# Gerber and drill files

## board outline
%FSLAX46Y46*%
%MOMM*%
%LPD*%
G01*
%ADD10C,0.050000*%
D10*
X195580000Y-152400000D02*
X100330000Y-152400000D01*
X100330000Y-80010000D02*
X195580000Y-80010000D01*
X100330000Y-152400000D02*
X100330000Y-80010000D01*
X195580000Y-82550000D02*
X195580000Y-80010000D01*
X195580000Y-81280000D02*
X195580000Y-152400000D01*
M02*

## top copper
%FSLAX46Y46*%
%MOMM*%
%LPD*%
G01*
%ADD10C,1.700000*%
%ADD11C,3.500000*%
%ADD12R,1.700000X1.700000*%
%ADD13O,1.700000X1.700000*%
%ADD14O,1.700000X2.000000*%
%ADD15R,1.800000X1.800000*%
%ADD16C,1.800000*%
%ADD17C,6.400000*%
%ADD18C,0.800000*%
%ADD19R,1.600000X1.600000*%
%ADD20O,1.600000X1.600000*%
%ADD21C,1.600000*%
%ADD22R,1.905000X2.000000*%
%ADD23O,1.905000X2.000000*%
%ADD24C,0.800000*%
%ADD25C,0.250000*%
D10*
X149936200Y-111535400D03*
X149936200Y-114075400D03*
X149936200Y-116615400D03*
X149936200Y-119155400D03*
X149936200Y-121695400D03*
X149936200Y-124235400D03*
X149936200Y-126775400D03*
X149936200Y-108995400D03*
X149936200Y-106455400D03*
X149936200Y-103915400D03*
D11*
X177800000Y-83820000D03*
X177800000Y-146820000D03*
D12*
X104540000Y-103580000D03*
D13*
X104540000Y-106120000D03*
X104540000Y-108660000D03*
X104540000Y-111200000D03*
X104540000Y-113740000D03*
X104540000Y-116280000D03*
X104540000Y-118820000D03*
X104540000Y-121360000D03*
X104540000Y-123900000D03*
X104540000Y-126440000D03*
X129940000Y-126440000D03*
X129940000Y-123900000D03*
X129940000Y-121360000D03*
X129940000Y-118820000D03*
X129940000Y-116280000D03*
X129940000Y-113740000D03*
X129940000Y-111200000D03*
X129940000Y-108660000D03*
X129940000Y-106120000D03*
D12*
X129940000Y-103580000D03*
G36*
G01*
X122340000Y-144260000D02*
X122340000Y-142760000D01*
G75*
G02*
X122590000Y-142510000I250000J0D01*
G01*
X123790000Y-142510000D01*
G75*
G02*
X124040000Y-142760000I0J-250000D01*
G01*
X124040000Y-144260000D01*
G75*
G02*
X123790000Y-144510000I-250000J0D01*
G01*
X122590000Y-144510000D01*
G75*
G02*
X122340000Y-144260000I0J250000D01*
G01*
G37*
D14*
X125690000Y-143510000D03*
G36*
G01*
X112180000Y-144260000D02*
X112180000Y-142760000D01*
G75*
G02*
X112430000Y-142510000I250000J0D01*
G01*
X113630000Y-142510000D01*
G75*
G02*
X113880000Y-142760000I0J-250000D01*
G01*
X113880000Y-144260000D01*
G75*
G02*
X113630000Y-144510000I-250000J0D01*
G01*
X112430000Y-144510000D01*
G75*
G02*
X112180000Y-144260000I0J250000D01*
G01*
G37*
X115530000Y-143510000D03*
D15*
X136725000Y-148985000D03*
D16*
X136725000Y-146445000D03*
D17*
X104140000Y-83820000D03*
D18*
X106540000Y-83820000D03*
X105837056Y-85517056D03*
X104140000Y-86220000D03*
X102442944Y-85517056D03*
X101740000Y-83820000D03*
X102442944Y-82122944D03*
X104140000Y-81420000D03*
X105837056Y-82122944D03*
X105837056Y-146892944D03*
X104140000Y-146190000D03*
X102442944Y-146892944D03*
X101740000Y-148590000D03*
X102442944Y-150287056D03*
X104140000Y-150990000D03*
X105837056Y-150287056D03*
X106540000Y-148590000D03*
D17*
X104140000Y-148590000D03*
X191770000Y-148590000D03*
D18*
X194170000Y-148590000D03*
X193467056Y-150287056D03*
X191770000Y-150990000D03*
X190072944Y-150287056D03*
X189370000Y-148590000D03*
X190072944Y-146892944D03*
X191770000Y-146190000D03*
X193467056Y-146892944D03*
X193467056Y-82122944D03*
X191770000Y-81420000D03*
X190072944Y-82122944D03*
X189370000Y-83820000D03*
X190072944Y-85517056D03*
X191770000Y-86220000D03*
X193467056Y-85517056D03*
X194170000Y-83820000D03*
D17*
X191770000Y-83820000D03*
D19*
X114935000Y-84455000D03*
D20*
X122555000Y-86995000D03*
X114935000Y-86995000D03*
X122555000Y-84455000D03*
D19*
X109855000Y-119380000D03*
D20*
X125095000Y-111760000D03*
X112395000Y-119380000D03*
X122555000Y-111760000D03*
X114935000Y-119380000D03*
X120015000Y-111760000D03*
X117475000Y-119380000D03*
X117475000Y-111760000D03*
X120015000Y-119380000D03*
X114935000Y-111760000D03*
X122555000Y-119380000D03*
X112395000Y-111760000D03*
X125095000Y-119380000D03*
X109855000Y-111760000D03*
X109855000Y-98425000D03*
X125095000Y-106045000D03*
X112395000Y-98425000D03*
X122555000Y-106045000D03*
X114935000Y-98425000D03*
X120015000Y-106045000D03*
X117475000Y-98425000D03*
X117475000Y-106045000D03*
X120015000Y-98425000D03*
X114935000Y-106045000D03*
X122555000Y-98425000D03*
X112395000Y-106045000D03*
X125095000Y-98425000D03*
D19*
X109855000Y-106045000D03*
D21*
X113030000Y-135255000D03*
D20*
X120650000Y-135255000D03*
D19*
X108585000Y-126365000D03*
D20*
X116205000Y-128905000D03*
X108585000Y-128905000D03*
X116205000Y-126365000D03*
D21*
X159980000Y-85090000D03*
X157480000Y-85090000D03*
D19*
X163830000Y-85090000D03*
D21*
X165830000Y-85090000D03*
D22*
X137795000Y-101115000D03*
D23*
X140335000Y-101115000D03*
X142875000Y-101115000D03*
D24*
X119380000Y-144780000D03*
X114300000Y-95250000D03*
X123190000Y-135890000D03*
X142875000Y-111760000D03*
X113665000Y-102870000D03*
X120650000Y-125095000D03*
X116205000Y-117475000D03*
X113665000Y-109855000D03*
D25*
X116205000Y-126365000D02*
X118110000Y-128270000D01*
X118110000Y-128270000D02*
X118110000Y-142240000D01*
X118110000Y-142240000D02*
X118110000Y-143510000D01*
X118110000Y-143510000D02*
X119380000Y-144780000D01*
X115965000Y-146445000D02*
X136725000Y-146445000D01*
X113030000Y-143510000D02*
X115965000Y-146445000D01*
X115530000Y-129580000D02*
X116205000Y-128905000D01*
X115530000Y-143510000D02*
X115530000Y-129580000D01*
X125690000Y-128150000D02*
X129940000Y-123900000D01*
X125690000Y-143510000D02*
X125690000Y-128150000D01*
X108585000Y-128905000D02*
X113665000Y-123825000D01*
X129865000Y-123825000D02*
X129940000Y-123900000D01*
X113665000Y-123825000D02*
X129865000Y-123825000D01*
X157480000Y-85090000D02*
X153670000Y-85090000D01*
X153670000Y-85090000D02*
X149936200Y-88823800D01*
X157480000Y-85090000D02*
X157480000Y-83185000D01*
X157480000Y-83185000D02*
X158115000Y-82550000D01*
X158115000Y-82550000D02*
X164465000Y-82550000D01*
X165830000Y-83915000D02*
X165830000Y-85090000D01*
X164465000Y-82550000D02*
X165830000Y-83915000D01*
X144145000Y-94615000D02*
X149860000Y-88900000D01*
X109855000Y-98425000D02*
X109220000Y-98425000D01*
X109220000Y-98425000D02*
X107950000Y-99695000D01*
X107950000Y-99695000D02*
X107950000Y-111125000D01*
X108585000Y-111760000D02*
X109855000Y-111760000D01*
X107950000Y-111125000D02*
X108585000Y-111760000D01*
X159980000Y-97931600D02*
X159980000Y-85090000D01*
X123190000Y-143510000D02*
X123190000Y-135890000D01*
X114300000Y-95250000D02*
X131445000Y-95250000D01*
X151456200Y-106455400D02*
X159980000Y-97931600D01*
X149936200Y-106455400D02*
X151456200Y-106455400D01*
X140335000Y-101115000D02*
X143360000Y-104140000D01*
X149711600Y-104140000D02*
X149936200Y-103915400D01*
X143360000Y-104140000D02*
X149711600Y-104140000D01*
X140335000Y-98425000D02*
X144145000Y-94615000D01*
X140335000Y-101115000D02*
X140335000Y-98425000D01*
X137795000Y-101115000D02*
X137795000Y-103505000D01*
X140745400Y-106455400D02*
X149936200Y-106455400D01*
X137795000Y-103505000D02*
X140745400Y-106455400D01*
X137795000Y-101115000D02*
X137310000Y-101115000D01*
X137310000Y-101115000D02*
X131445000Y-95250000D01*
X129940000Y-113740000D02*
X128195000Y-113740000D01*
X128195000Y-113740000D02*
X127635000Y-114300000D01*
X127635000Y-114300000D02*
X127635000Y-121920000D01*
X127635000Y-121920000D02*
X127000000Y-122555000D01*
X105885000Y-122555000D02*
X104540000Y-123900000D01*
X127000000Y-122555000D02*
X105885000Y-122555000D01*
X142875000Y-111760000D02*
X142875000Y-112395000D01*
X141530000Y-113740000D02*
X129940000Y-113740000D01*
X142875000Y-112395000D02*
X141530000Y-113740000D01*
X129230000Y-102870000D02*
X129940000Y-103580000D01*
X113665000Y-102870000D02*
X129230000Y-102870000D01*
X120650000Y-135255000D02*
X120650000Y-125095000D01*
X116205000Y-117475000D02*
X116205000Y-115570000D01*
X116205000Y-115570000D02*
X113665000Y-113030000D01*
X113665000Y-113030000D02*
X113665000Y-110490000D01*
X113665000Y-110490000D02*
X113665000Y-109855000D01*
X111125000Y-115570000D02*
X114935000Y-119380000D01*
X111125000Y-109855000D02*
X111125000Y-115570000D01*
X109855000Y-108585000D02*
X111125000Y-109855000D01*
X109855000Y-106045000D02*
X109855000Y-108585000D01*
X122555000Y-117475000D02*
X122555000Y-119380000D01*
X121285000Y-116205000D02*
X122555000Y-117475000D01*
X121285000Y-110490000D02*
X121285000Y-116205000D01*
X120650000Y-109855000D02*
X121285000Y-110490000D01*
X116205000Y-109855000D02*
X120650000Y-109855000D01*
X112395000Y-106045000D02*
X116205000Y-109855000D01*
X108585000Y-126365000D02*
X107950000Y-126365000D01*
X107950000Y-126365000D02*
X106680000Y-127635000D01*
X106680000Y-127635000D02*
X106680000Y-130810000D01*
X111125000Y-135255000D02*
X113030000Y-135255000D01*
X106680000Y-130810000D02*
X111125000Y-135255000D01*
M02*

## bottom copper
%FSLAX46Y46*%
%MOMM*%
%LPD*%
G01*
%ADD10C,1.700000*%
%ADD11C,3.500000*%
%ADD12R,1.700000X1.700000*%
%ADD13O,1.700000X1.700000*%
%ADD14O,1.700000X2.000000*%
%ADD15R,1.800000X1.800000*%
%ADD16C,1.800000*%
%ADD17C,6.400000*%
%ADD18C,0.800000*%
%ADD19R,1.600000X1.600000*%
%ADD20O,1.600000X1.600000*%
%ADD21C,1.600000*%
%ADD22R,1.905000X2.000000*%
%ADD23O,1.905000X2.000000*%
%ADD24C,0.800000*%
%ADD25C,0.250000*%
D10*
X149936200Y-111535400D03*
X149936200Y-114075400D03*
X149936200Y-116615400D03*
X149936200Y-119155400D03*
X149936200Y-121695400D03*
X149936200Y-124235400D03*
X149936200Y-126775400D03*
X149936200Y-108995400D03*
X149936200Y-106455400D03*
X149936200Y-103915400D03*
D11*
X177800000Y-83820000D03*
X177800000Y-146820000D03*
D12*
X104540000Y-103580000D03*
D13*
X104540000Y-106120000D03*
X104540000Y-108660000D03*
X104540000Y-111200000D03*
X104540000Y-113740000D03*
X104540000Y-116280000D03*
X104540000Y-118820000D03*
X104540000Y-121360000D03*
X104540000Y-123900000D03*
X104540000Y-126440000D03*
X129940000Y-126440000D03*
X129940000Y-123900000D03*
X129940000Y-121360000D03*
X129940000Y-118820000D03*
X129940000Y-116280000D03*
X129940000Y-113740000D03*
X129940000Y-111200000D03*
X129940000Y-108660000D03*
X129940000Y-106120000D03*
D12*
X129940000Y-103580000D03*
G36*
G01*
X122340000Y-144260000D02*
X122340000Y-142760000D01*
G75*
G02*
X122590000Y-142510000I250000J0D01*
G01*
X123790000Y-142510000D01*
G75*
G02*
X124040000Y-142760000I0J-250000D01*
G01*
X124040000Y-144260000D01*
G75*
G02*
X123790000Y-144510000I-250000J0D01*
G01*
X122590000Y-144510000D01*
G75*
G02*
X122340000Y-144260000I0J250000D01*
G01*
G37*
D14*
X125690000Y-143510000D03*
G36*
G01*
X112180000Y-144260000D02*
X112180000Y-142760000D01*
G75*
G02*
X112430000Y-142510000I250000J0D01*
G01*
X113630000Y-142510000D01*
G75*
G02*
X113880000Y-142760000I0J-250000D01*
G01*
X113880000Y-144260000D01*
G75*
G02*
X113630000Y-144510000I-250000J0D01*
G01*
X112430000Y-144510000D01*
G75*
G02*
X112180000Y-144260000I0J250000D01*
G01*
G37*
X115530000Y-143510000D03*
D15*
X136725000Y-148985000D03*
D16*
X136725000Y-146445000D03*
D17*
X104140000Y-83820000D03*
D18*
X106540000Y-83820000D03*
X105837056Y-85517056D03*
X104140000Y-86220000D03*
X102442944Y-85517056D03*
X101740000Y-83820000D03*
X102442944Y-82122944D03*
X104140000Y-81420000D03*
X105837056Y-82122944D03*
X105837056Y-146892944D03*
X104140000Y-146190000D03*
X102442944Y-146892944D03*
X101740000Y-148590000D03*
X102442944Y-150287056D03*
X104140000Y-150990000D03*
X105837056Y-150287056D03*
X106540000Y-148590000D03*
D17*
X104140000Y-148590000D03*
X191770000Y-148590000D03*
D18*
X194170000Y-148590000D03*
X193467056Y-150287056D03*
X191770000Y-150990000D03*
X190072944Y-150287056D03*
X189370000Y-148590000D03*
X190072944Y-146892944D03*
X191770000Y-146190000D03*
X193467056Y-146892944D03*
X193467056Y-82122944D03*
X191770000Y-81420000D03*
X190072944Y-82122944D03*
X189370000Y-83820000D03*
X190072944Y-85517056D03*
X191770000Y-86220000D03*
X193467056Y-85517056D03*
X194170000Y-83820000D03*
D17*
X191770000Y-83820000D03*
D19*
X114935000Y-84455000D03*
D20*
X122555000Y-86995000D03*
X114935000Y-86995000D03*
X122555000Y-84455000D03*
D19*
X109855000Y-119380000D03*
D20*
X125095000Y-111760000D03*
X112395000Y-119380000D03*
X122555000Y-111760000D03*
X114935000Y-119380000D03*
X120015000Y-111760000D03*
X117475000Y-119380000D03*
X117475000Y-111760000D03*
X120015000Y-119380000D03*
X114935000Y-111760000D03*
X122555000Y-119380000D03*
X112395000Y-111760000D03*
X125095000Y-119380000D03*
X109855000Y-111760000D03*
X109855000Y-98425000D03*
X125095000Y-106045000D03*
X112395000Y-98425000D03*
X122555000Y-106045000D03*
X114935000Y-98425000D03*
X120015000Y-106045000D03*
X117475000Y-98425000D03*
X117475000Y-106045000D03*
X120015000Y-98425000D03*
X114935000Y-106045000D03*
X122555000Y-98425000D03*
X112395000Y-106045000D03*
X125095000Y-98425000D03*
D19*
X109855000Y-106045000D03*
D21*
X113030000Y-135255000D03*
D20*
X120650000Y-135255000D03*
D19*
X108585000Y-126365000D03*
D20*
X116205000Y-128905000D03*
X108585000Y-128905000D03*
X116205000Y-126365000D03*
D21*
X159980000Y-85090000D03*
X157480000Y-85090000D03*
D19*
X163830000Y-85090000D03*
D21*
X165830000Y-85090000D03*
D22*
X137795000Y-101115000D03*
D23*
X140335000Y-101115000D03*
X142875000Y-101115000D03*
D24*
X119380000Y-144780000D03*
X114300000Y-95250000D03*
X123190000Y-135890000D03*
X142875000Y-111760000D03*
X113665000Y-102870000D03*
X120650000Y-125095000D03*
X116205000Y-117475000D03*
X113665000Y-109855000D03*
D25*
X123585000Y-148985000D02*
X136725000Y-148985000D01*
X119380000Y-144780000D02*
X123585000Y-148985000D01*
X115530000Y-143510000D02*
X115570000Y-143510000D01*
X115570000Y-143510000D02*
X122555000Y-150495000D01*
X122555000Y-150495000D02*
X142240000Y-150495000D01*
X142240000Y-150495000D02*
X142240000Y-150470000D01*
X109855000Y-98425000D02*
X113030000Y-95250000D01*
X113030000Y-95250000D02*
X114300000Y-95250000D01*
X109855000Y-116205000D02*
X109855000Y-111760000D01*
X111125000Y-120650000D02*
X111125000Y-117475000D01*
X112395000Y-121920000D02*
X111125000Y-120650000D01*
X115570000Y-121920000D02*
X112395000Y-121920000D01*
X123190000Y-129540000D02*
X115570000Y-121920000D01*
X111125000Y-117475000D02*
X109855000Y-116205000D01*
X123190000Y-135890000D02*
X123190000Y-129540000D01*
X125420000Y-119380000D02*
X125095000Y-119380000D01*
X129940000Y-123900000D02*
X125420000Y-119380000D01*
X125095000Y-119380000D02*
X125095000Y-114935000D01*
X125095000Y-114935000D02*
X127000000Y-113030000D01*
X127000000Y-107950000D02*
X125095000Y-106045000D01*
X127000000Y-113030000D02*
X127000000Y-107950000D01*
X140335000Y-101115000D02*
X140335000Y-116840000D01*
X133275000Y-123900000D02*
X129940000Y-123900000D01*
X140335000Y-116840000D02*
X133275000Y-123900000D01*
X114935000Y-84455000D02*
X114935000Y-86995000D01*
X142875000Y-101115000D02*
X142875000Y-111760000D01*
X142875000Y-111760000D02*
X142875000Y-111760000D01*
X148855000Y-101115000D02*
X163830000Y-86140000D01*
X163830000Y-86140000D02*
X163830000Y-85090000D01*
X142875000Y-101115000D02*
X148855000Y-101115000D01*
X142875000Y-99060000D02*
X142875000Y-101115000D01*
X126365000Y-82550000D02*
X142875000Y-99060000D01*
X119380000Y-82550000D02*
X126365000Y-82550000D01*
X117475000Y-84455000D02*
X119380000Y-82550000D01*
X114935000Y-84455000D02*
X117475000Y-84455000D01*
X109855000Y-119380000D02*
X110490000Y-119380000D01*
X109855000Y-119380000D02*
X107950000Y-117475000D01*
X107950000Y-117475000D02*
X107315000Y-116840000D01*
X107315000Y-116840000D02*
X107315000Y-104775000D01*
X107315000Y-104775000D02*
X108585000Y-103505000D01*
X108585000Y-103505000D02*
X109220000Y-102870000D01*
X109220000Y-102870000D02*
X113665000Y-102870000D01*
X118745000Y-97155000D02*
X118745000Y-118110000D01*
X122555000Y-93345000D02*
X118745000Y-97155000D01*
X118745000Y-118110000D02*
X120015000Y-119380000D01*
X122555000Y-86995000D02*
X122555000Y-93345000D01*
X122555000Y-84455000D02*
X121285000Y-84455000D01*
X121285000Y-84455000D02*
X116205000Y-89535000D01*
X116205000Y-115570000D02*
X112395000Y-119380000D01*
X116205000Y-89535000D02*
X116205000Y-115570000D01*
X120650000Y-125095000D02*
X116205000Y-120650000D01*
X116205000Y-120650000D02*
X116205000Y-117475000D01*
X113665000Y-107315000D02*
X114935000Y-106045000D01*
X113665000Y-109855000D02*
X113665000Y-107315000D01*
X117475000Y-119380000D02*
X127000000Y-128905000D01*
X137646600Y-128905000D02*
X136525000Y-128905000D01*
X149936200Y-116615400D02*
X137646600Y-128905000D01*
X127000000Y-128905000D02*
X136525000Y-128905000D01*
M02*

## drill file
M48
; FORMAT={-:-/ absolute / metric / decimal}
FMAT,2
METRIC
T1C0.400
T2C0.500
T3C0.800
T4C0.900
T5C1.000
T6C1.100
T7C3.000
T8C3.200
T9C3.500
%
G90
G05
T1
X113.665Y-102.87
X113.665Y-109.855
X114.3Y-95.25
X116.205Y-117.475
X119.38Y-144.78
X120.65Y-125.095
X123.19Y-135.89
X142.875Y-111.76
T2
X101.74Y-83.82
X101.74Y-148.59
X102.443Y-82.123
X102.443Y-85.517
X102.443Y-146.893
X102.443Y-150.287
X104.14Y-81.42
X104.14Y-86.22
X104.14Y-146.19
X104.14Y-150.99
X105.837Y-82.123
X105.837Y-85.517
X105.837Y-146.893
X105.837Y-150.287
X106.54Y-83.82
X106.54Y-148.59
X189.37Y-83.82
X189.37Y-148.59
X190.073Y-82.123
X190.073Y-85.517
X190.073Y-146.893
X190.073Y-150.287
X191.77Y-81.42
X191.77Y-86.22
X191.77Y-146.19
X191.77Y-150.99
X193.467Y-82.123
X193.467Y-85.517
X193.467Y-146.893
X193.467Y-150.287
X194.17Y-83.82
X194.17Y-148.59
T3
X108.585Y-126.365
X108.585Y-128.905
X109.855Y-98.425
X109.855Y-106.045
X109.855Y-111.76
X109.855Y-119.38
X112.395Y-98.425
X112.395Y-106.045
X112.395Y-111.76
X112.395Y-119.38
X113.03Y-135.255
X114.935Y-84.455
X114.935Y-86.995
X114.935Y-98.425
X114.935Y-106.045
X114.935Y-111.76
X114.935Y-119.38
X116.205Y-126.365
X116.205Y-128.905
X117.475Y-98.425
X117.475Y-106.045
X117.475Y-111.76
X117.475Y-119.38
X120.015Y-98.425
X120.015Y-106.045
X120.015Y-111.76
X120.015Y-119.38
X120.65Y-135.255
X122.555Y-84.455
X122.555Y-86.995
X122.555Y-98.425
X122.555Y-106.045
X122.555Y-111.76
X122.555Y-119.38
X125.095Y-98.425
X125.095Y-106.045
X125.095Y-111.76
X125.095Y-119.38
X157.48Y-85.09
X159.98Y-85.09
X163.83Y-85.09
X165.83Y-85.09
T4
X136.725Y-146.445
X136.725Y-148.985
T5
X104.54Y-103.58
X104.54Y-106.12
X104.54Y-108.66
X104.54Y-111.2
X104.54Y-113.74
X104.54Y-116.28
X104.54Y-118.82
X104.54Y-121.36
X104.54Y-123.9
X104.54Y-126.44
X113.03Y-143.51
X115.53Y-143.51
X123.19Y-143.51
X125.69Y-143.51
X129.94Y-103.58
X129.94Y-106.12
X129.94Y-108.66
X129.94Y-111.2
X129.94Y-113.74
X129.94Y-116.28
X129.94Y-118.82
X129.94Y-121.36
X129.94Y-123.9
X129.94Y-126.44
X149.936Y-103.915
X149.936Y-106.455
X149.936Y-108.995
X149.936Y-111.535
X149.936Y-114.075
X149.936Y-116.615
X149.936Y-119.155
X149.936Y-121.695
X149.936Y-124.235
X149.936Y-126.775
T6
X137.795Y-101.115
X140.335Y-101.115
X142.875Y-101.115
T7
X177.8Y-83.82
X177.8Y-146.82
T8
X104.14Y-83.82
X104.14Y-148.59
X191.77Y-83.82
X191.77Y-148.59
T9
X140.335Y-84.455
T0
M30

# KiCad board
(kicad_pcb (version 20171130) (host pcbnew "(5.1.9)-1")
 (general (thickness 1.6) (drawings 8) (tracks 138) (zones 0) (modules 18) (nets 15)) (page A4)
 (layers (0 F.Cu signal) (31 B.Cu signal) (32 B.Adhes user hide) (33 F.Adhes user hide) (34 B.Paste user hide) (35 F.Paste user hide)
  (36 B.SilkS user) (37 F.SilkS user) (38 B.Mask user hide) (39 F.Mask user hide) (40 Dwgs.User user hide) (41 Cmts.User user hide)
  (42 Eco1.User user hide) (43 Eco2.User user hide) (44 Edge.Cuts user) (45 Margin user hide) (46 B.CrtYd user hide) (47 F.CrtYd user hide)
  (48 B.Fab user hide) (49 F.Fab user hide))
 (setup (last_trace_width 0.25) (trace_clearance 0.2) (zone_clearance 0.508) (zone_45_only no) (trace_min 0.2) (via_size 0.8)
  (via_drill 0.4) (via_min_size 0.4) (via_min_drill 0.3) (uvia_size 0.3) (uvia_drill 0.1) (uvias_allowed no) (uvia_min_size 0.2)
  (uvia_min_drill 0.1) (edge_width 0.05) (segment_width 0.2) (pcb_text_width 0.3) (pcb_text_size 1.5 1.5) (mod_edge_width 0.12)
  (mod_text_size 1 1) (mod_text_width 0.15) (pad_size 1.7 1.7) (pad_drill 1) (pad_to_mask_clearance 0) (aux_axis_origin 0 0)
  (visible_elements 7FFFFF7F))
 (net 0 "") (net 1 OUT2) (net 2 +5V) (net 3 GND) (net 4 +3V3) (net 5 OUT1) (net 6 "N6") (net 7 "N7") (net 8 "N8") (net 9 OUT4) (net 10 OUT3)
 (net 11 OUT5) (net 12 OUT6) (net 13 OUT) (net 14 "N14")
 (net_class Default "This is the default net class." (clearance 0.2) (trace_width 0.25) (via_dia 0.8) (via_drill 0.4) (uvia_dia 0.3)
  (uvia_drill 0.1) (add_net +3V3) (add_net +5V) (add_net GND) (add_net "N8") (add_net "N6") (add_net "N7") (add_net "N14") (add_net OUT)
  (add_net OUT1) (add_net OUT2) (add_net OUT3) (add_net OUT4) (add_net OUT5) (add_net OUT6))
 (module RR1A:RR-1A (layer F.Cu) (at 177.8 115.32 270)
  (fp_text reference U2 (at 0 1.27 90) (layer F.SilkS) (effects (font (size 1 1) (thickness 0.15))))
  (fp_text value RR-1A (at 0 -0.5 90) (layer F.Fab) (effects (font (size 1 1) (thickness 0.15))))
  (pad 4 thru_hole circle (at -3.7846 27.8638 270) (size 1.7 1.7) (drill 1) (layers *.Cu *.Mask))
  (pad 5 thru_hole circle (at -1.2446 27.8638 270) (size 1.7 1.7) (drill 1) (layers *.Cu *.Mask))
  (pad 6 thru_hole circle (at 1.2954 27.8638 270) (size 1.7 1.7) (drill 1) (layers *.Cu *.Mask) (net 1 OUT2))
  (pad 7 thru_hole circle (at 3.8354 27.8638 270) (size 1.7 1.7) (drill 1) (layers *.Cu *.Mask))
  (pad 8 thru_hole circle (at 6.3754 27.8638 270) (size 1.7 1.7) (drill 1) (layers *.Cu *.Mask))
  (pad 9 thru_hole circle (at 8.9154 27.8638 270) (size 1.7 1.7) (drill 1) (layers *.Cu *.Mask))
  (pad 10 thru_hole circle (at 11.4554 27.8638 270) (size 1.7 1.7) (drill 1) (layers *.Cu *.Mask))
  (pad 3 thru_hole circle (at -6.3246 27.8638 270) (size 1.7 1.7) (drill 1) (layers *.Cu *.Mask))
  (pad 2 thru_hole circle (at -8.8646 27.8638 270) (size 1.7 1.7) (drill 1) (layers *.Cu *.Mask) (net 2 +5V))
  (pad 1 thru_hole circle (at -11.4046 27.8638 270) (size 1.7 1.7) (drill 1) (layers *.Cu *.Mask) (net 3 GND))
  (pad 11 thru_hole circle (at -31.5 0 270) (size 3.5 3.5) (drill 3) (layers *.Cu *.Mask))
  (pad 12 thru_hole circle (at 31.5 0 270) (size 3.5 3.5) (drill 3) (layers *.Cu *.Mask)))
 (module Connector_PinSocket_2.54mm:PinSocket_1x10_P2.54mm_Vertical (layer F.Cu) (at 104.54 103.58)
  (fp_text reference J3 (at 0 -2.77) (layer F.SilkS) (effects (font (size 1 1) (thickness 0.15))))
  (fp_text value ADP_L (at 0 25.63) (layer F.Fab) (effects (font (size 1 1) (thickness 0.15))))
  (pad 1 thru_hole rect (at 0 0) (size 1.7 1.7) (drill 1) (layers *.Cu *.Mask))
  (pad 2 thru_hole oval (at 0 2.54) (size 1.7 1.7) (drill 1) (layers *.Cu *.Mask))
  (pad 3 thru_hole oval (at 0 5.08) (size 1.7 1.7) (drill 1) (layers *.Cu *.Mask))
  (pad 4 thru_hole oval (at 0 7.62) (size 1.7 1.7) (drill 1) (layers *.Cu *.Mask))
  (pad 5 thru_hole oval (at 0 10.16) (size 1.7 1.7) (drill 1) (layers *.Cu *.Mask))
  (pad 6 thru_hole oval (at 0 12.7) (size 1.7 1.7) (drill 1) (layers *.Cu *.Mask))
  (pad 7 thru_hole oval (at 0 15.24) (size 1.7 1.7) (drill 1) (layers *.Cu *.Mask))
  (pad 8 thru_hole oval (at 0 17.78) (size 1.7 1.7) (drill 1) (layers *.Cu *.Mask))
  (pad 9 thru_hole oval (at 0 20.32) (size 1.7 1.7) (drill 1) (layers *.Cu *.Mask) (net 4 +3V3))
  (pad 10 thru_hole oval (at 0 22.86) (size 1.7 1.7) (drill 1) (layers *.Cu *.Mask)))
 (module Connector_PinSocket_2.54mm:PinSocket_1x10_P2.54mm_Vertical (layer F.Cu) (at 129.94 103.58)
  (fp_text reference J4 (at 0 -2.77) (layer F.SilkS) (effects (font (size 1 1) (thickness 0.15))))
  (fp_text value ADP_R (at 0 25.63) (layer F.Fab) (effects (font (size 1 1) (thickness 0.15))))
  (pad 10 thru_hole oval (at 0 22.86) (size 1.7 1.7) (drill 1) (layers *.Cu *.Mask))
  (pad 9 thru_hole oval (at 0 20.32) (size 1.7 1.7) (drill 1) (layers *.Cu *.Mask) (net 3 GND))
  (pad 8 thru_hole oval (at 0 17.78) (size 1.7 1.7) (drill 1) (layers *.Cu *.Mask))
  (pad 7 thru_hole oval (at 0 15.24) (size 1.7 1.7) (drill 1) (layers *.Cu *.Mask))
  (pad 6 thru_hole oval (at 0 12.7) (size 1.7 1.7) (drill 1) (layers *.Cu *.Mask))
  (pad 5 thru_hole oval (at 0 10.16) (size 1.7 1.7) (drill 1) (layers *.Cu *.Mask) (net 4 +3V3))
  (pad 4 thru_hole oval (at 0 7.62) (size 1.7 1.7) (drill 1) (layers *.Cu *.Mask))
  (pad 3 thru_hole oval (at 0 5.08) (size 1.7 1.7) (drill 1) (layers *.Cu *.Mask))
  (pad 2 thru_hole oval (at 0 2.54) (size 1.7 1.7) (drill 1) (layers *.Cu *.Mask))
  (pad 1 thru_hole rect (at 0 0) (size 1.7 1.7) (drill 1) (layers *.Cu *.Mask) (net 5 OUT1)))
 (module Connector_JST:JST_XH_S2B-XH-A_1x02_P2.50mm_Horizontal (layer F.Cu) (at 123.19 143.51)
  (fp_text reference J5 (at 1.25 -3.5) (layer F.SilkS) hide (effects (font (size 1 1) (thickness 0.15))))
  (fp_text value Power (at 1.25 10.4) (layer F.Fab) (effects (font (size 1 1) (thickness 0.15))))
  (pad 1 thru_hole roundrect (at 0 0) (size 1.7 2) (drill 1) (layers *.Cu *.Mask) (roundrect_rratio 0.1470588235294118) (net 2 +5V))
  (pad 2 thru_hole oval (at 2.5 0) (size 1.7 2) (drill 1) (layers *.Cu *.Mask) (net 3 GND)))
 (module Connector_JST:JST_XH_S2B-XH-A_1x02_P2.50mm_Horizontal (layer F.Cu) (at 113.03 143.51)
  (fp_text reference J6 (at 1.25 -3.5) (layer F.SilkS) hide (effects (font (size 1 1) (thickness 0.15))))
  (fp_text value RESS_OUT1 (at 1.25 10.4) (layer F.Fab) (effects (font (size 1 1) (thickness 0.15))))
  (pad 1 thru_hole roundrect (at 0 0) (size 1.7 2) (drill 1) (layers *.Cu *.Mask) (roundrect_rratio 0.1470588235294118) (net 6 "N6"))
  (pad 2 thru_hole oval (at 2.5 0) (size 1.7 2) (drill 1) (layers *.Cu *.Mask) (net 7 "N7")))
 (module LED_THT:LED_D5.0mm (layer F.Cu) (at 136.725 148.985 90)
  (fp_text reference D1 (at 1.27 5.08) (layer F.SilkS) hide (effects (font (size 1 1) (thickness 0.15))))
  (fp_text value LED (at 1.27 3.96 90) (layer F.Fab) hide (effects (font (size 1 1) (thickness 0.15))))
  (pad 1 thru_hole rect (at 0 0 90) (size 1.8 1.8) (drill 0.9) (layers *.Cu *.Mask) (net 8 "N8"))
  (pad 2 thru_hole circle (at 2.54 0 90) (size 1.8 1.8) (drill 0.9) (layers *.Cu *.Mask) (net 6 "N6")))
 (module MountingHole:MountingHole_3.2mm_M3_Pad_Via (layer F.Cu) (at 104.14 83.82)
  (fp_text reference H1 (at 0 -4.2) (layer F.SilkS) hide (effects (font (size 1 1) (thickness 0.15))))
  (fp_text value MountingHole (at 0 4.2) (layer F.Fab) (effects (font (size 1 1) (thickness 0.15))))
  (pad 1 thru_hole circle (at 0 0) (size 6.4 6.4) (drill 3.2) (layers *.Cu *.Mask))
  (pad 1 thru_hole circle (at 2.4 0) (size 0.8 0.8) (drill 0.5) (layers *.Cu *.Mask))
  (pad 1 thru_hole circle (at 1.697056 1.697056) (size 0.8 0.8) (drill 0.5) (layers *.Cu *.Mask))
  (pad 1 thru_hole circle (at 0 2.4) (size 0.8 0.8) (drill 0.5) (layers *.Cu *.Mask))
  (pad 1 thru_hole circle (at -1.697056 1.697056) (size 0.8 0.8) (drill 0.5) (layers *.Cu *.Mask))
  (pad 1 thru_hole circle (at -2.4 0) (size 0.8 0.8) (drill 0.5) (layers *.Cu *.Mask))
  (pad 1 thru_hole circle (at -1.697056 -1.697056) (size 0.8 0.8) (drill 0.5) (layers *.Cu *.Mask))
  (pad 1 thru_hole circle (at 0 -2.4) (size 0.8 0.8) (drill 0.5) (layers *.Cu *.Mask))
  (pad 1 thru_hole circle (at 1.697056 -1.697056) (size 0.8 0.8) (drill 0.5) (layers *.Cu *.Mask)))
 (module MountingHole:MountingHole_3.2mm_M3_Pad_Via (layer F.Cu) (at 104.14 148.59)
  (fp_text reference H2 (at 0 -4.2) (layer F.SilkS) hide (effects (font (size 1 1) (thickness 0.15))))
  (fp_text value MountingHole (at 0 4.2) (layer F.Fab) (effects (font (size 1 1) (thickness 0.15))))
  (pad 1 thru_hole circle (at 1.697056 -1.697056) (size 0.8 0.8) (drill 0.5) (layers *.Cu *.Mask))
  (pad 1 thru_hole circle (at 0 -2.4) (size 0.8 0.8) (drill 0.5) (layers *.Cu *.Mask))
  (pad 1 thru_hole circle (at -1.697056 -1.697056) (size 0.8 0.8) (drill 0.5) (layers *.Cu *.Mask))
  (pad 1 thru_hole circle (at -2.4 0) (size 0.8 0.8) (drill 0.5) (layers *.Cu *.Mask))
  (pad 1 thru_hole circle (at -1.697056 1.697056) (size 0.8 0.8) (drill 0.5) (layers *.Cu *.Mask))
  (pad 1 thru_hole circle (at 0 2.4) (size 0.8 0.8) (drill 0.5) (layers *.Cu *.Mask))
  (pad 1 thru_hole circle (at 1.697056 1.697056) (size 0.8 0.8) (drill 0.5) (layers *.Cu *.Mask))
  (pad 1 thru_hole circle (at 2.4 0) (size 0.8 0.8) (drill 0.5) (layers *.Cu *.Mask))
  (pad 1 thru_hole circle (at 0 0) (size 6.4 6.4) (drill 3.2) (layers *.Cu *.Mask)))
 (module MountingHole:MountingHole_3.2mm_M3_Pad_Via (layer F.Cu) (at 191.77 148.59)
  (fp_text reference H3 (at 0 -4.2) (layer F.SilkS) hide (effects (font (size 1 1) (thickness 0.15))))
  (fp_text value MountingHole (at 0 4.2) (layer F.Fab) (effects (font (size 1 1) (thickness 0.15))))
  (pad 1 thru_hole circle (at 0 0) (size 6.4 6.4) (drill 3.2) (layers *.Cu *.Mask))
  (pad 1 thru_hole circle (at 2.4 0) (size 0.8 0.8) (drill 0.5) (layers *.Cu *.Mask))
  (pad 1 thru_hole circle (at 1.697056 1.697056) (size 0.8 0.8) (drill 0.5) (layers *.Cu *.Mask))
  (pad 1 thru_hole circle (at 0 2.4) (size 0.8 0.8) (drill 0.5) (layers *.Cu *.Mask))
  (pad 1 thru_hole circle (at -1.697056 1.697056) (size 0.8 0.8) (drill 0.5) (layers *.Cu *.Mask))
  (pad 1 thru_hole circle (at -2.4 0) (size 0.8 0.8) (drill 0.5) (layers *.Cu *.Mask))
  (pad 1 thru_hole circle (at -1.697056 -1.697056) (size 0.8 0.8) (drill 0.5) (layers *.Cu *.Mask))
  (pad 1 thru_hole circle (at 0 -2.4) (size 0.8 0.8) (drill 0.5) (layers *.Cu *.Mask))
  (pad 1 thru_hole circle (at 1.697056 -1.697056) (size 0.8 0.8) (drill 0.5) (layers *.Cu *.Mask)))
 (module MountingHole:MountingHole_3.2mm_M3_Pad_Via (layer F.Cu) (at 191.77 83.82)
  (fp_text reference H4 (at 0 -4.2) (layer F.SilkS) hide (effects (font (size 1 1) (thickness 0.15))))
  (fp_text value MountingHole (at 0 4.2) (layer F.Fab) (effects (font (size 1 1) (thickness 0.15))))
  (pad 1 thru_hole circle (at 1.697056 -1.697056) (size 0.8 0.8) (drill 0.5) (layers *.Cu *.Mask))
  (pad 1 thru_hole circle (at 0 -2.4) (size 0.8 0.8) (drill 0.5) (layers *.Cu *.Mask))
  (pad 1 thru_hole circle (at -1.697056 -1.697056) (size 0.8 0.8) (drill 0.5) (layers *.Cu *.Mask))
  (pad 1 thru_hole circle (at -2.4 0) (size 0.8 0.8) (drill 0.5) (layers *.Cu *.Mask))
  (pad 1 thru_hole circle (at -1.697056 1.697056) (size 0.8 0.8) (drill 0.5) (layers *.Cu *.Mask))
  (pad 1 thru_hole circle (at 0 2.4) (size 0.8 0.8) (drill 0.5) (layers *.Cu *.Mask))
  (pad 1 thru_hole circle (at 1.697056 1.697056) (size 0.8 0.8) (drill 0.5) (layers *.Cu *.Mask))
  (pad 1 thru_hole circle (at 2.4 0) (size 0.8 0.8) (drill 0.5) (layers *.Cu *.Mask))
  (pad 1 thru_hole circle (at 0 0) (size 6.4 6.4) (drill 3.2) (layers *.Cu *.Mask)))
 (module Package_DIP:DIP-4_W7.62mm (layer F.Cu) (at 114.935 84.455)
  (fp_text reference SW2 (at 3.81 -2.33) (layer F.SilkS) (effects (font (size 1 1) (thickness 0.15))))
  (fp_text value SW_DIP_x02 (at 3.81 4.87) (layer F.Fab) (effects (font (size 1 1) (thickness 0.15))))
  (pad 1 thru_hole rect (at 0 0) (size 1.6 1.6) (drill 0.8) (layers *.Cu *.Mask) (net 4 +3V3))
  (pad 3 thru_hole oval (at 7.62 2.54) (size 1.6 1.6) (drill 0.8) (layers *.Cu *.Mask) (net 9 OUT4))
  (pad 2 thru_hole oval (at 0 2.54) (size 1.6 1.6) (drill 0.8) (layers *.Cu *.Mask) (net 4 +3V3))
  (pad 4 thru_hole oval (at 7.62 0) (size 1.6 1.6) (drill 0.8) (layers *.Cu *.Mask) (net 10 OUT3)))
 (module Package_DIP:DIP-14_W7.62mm (layer F.Cu) (at 109.855 119.38 90)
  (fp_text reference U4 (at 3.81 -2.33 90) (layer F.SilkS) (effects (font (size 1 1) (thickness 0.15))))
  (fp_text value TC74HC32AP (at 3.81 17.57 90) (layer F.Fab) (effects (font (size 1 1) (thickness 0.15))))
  (pad 1 thru_hole rect (at 0 0 90) (size 1.6 1.6) (drill 0.8) (layers *.Cu *.Mask) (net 5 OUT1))
  (pad 8 thru_hole oval (at 7.62 15.24 90) (size 1.6 1.6) (drill 0.8) (layers *.Cu *.Mask))
  (pad 2 thru_hole oval (at 0 2.54 90) (size 1.6 1.6) (drill 0.8) (layers *.Cu *.Mask) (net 10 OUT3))
  (pad 9 thru_hole oval (at 7.62 12.7 90) (size 1.6 1.6) (drill 0.8) (layers *.Cu *.Mask))
  (pad 3 thru_hole oval (at 0 5.08 90) (size 1.6 1.6) (drill 0.8) (layers *.Cu *.Mask) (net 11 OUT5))
  (pad 10 thru_hole oval (at 7.62 10.16 90) (size 1.6 1.6) (drill 0.8) (layers *.Cu *.Mask))
  (pad 4 thru_hole oval (at 0 7.62 90) (size 1.6 1.6) (drill 0.8) (layers *.Cu *.Mask) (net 1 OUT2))
  (pad 11 thru_hole oval (at 7.62 7.62 90) (size 1.6 1.6) (drill 0.8) (layers *.Cu *.Mask))
  (pad 5 thru_hole oval (at 0 10.16 90) (size 1.6 1.6) (drill 0.8) (layers *.Cu *.Mask) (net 9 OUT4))
  (pad 12 thru_hole oval (at 7.62 5.08 90) (size 1.6 1.6) (drill 0.8) (layers *.Cu *.Mask))
  (pad 6 thru_hole oval (at 0 12.7 90) (size 1.6 1.6) (drill 0.8) (layers *.Cu *.Mask) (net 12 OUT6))
  (pad 13 thru_hole oval (at 7.62 2.54 90) (size 1.6 1.6) (drill 0.8) (layers *.Cu *.Mask))
  (pad 7 thru_hole oval (at 0 15.24 90) (size 1.6 1.6) (drill 0.8) (layers *.Cu *.Mask) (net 3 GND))
  (pad 14 thru_hole oval (at 7.62 0 90) (size 1.6 1.6) (drill 0.8) (layers *.Cu *.Mask) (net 2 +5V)))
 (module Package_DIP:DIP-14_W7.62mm (layer F.Cu) (at 109.855 106.045 90)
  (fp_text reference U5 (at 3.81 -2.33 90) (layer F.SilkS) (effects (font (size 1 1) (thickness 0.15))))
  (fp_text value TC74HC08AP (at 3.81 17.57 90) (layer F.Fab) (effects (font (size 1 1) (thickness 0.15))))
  (pad 14 thru_hole oval (at 7.62 0 90) (size 1.6 1.6) (drill 0.8) (layers *.Cu *.Mask) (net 2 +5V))
  (pad 7 thru_hole oval (at 0 15.24 90) (size 1.6 1.6) (drill 0.8) (layers *.Cu *.Mask) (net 3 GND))
  (pad 13 thru_hole oval (at 7.62 2.54 90) (size 1.6 1.6) (drill 0.8) (layers *.Cu *.Mask))
  (pad 6 thru_hole oval (at 0 12.7 90) (size 1.6 1.6) (drill 0.8) (layers *.Cu *.Mask))
  (pad 12 thru_hole oval (at 7.62 5.08 90) (size 1.6 1.6) (drill 0.8) (layers *.Cu *.Mask))
  (pad 5 thru_hole oval (at 0 10.16 90) (size 1.6 1.6) (drill 0.8) (layers *.Cu *.Mask))
  (pad 11 thru_hole oval (at 7.62 7.62 90) (size 1.6 1.6) (drill 0.8) (layers *.Cu *.Mask))
  (pad 4 thru_hole oval (at 0 7.62 90) (size 1.6 1.6) (drill 0.8) (layers *.Cu *.Mask))
  (pad 10 thru_hole oval (at 7.62 10.16 90) (size 1.6 1.6) (drill 0.8) (layers *.Cu *.Mask))
  (pad 3 thru_hole oval (at 0 5.08 90) (size 1.6 1.6) (drill 0.8) (layers *.Cu *.Mask) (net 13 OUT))
  (pad 9 thru_hole oval (at 7.62 12.7 90) (size 1.6 1.6) (drill 0.8) (layers *.Cu *.Mask))
  (pad 2 thru_hole oval (at 0 2.54 90) (size 1.6 1.6) (drill 0.8) (layers *.Cu *.Mask) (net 12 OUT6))
  (pad 8 thru_hole oval (at 7.62 15.24 90) (size 1.6 1.6) (drill 0.8) (layers *.Cu *.Mask))
  (pad 1 thru_hole rect (at 0 0 90) (size 1.6 1.6) (drill 0.8) (layers *.Cu *.Mask) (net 11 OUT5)))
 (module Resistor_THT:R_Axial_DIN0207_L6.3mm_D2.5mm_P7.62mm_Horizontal (layer F.Cu) (at 113.03 135.255)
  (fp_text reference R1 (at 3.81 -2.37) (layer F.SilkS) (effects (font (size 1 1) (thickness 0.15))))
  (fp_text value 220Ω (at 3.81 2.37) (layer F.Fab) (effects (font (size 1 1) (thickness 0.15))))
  (pad 1 thru_hole circle (at 0 0) (size 1.6 1.6) (drill 0.8) (layers *.Cu *.Mask) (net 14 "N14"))
  (pad 2 thru_hole oval (at 7.62 0) (size 1.6 1.6) (drill 0.8) (layers *.Cu *.Mask) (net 13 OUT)))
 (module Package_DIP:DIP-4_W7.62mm (layer F.Cu) (at 108.585 126.365)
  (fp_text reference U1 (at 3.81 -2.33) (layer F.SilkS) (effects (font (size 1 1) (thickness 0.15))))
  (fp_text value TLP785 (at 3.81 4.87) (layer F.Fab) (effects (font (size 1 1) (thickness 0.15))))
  (pad 1 thru_hole rect (at 0 0) (size 1.6 1.6) (drill 0.8) (layers *.Cu *.Mask) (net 14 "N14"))
  (pad 3 thru_hole oval (at 7.62 2.54) (size 1.6 1.6) (drill 0.8) (layers *.Cu *.Mask) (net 7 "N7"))
  (pad 2 thru_hole oval (at 0 2.54) (size 1.6 1.6) (drill 0.8) (layers *.Cu *.Mask) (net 3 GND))
  (pad 4 thru_hole oval (at 7.62 0) (size 1.6 1.6) (drill 0.8) (layers *.Cu *.Mask) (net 8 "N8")))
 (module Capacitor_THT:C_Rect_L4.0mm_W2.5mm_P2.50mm (layer F.Cu) (at 159.98 85.09 180)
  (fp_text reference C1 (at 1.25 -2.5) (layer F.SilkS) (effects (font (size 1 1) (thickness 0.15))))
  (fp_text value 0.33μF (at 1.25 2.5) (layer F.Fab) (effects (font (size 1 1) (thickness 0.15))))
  (pad 1 thru_hole circle (at 0 0 180) (size 1.6 1.6) (drill 0.8) (layers *.Cu *.Mask) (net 2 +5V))
  (pad 2 thru_hole circle (at 2.5 0 180) (size 1.6 1.6) (drill 0.8) (layers *.Cu *.Mask) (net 3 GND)))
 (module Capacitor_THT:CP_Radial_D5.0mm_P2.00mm (layer F.Cu) (at 163.83 85.09)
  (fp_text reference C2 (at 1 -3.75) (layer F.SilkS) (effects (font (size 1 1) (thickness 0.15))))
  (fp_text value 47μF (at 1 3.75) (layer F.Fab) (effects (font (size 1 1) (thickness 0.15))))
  (pad 1 thru_hole rect (at 0 0) (size 1.6 1.6) (drill 0.8) (layers *.Cu *.Mask) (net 4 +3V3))
  (pad 2 thru_hole circle (at 2 0) (size 1.6 1.6) (drill 0.8) (layers *.Cu *.Mask) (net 3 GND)))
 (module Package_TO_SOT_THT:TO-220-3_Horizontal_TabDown (layer F.Cu) (at 137.795 101.115)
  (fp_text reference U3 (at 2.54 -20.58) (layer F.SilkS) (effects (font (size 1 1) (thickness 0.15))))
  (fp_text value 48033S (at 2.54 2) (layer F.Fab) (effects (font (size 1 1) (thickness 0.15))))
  (pad "" np_thru_hole oval (at 2.54 -16.66) (size 3.5 3.5) (drill 3.5) (layers *.Cu *.Mask))
  (pad 1 thru_hole rect (at 0 0) (size 1.905 2) (drill 1.1) (layers *.Cu *.Mask) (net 2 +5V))
  (pad 2 thru_hole oval (at 2.54 0) (size 1.905 2) (drill 1.1) (layers *.Cu *.Mask) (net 3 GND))
  (pad 3 thru_hole oval (at 5.08 0) (size 1.905 2) (drill 1.1) (layers *.Cu *.Mask) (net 4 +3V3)))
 (gr_line (start 195.58 152.4) (end 100.33 152.4) (layer Edge.Cuts) (width 0.05))
 (gr_line (start 100.33 80.01) (end 195.58 80.01) (layer Edge.Cuts) (width 0.05))
 (gr_line (start 100.33 152.4) (end 100.33 80.01) (layer Edge.Cuts) (width 0.05))
 (gr_line (start 195.58 82.55) (end 195.58 80.01) (layer Edge.Cuts) (width 0.05))
 (gr_line (start 195.58 81.28) (end 195.58 152.4) (layer Edge.Cuts) (width 0.05))
 (segment (start 116.205 126.365) (end 118.11 128.27) (width 0.25) (layer F.Cu) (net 8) (status 10))
 (segment (start 118.11 128.27) (end 118.11 142.24) (width 0.25) (layer F.Cu) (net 8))
 (segment (start 118.11 142.24) (end 118.11 143.51) (width 0.25) (layer F.Cu) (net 8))
 (segment (start 118.11 143.51) (end 119.38 144.78) (width 0.25) (layer F.Cu) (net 8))
 (via (at 119.38 144.78) (size 0.8) (drill 0.4) (layers F.Cu B.Cu) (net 8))
 (segment (start 123.585 148.985) (end 136.725 148.985) (width 0.25) (layer B.Cu) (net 8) (status 20))
 (segment (start 119.38 144.78) (end 123.585 148.985) (width 0.25) (layer B.Cu) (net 8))
 (segment (start 115.965 146.445) (end 136.725 146.445) (width 0.25) (layer F.Cu) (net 6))
 (segment (start 113.03 143.51) (end 115.965 146.445) (width 0.25) (layer F.Cu) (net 6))
 (segment (start 115.53 143.51) (end 115.57 143.51) (width 0.25) (layer B.Cu) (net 7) (status 30))
 (segment (start 115.57 143.51) (end 122.555 150.495) (width 0.25) (layer B.Cu) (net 7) (status 10))
 (segment (start 122.555 150.495) (end 142.24 150.495) (width 0.25) (layer B.Cu) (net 7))
 (segment (start 142.24 150.495) (end 142.24 150.47) (width 0.25) (layer B.Cu) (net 7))
 (segment (start 115.53 129.58) (end 116.205 128.905) (width 0.25) (layer F.Cu) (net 7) (status 20))
 (segment (start 115.53 143.51) (end 115.53 129.58) (width 0.25) (layer F.Cu) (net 7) (status 10))
 (segment (start 125.69 128.15) (end 129.94 123.9) (width 0.25) (layer F.Cu) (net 3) (status 20))
 (segment (start 125.69 143.51) (end 125.69 128.15) (width 0.25) (layer F.Cu) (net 3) (status 10))
 (segment (start 108.585 128.905) (end 113.665 123.825) (width 0.25) (layer F.Cu) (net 3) (status 10))
 (segment (start 129.865 123.825) (end 129.94 123.9) (width 0.25) (layer F.Cu) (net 3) (status 30))
 (segment (start 113.665 123.825) (end 129.865 123.825) (width 0.25) (layer F.Cu) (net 3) (status 20))
 (segment (start 157.48 85.09) (end 153.67 85.09) (width 0.25) (layer F.Cu) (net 3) (status 10))
 (segment (start 153.67 85.09) (end 149.9362 88.8238) (width 0.25) (layer F.Cu) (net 3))
 (segment (start 157.48 85.09) (end 157.48 83.185) (width 0.25) (layer F.Cu) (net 3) (status 10))
 (segment (start 157.48 83.185) (end 158.115 82.55) (width 0.25) (layer F.Cu) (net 3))
 (segment (start 158.115 82.55) (end 164.465 82.55) (width 0.25) (layer F.Cu) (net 3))
 (segment (start 165.83 83.915) (end 165.83 85.09) (width 0.25) (layer F.Cu) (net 3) (status 20))
 (segment (start 164.465 82.55) (end 165.83 83.915) (width 0.25) (layer F.Cu) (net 3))
 (segment (start 144.145 94.615) (end 149.86 88.9) (width 0.25) (layer F.Cu) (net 3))
 (segment (start 109.855 98.425) (end 109.22 98.425) (width 0.25) (layer F.Cu) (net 2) (status 30))
 (segment (start 109.22 98.425) (end 107.95 99.695) (width 0.25) (layer F.Cu) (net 2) (status 10))
 (segment (start 107.95 99.695) (end 107.95 111.125) (width 0.25) (layer F.Cu) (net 2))
 (segment (start 108.585 111.76) (end 109.855 111.76) (width 0.25) (layer F.Cu) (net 2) (status 20))
 (segment (start 107.95 111.125) (end 108.585 111.76) (width 0.25) (layer F.Cu) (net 2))
 (segment (start 159.98 97.9316) (end 159.98 85.09) (width 0.25) (layer F.Cu) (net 2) (status 20))
 (segment (start 109.855 98.425) (end 113.03 95.25) (width 0.25) (layer B.Cu) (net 2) (status 10))
 (segment (start 113.03 95.25) (end 114.3 95.25) (width 0.25) (layer B.Cu) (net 2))
 (via (at 114.3 95.25) (size 0.8) (drill 0.4) (layers F.Cu B.Cu) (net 2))
 (segment (start 123.19 143.51) (end 123.19 135.89) (width 0.25) (layer F.Cu) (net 2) (status 10))
 (via (at 123.19 135.89) (size 0.8) (drill 0.4) (layers F.Cu B.Cu) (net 2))
 (segment (start 109.855 116.205) (end 109.855 111.76) (width 0.25) (layer B.Cu) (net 2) (status 20))
 (segment (start 111.125 120.65) (end 111.125 117.475) (width 0.25) (layer B.Cu) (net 2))
 (segment (start 112.395 121.92) (end 111.125 120.65) (width 0.25) (layer B.Cu) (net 2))
 (segment (start 115.57 121.92) (end 112.395 121.92) (width 0.25) (layer B.Cu) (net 2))
 (segment (start 123.19 129.54) (end 115.57 121.92) (width 0.25) (layer B.Cu) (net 2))
 (segment (start 111.125 117.475) (end 109.855 116.205) (width 0.25) (layer B.Cu) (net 2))
 (segment (start 123.19 135.89) (end 123.19 129.54) (width 0.25) (layer B.Cu) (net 2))
 (segment (start 114.3 95.25) (end 131.445 95.25) (width 0.25) (layer F.Cu) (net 2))
 (segment (start 151.4562 106.4554) (end 159.98 97.9316) (width 0.25) (layer F.Cu) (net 2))
 (segment (start 149.9362 106.4554) (end 151.4562 106.4554) (width 0.25) (layer F.Cu) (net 2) (status 10))
 (segment (start 125.42 119.38) (end 125.095 119.38) (width 0.25) (layer B.Cu) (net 3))
 (segment (start 129.94 123.9) (end 125.42 119.38) (width 0.25) (layer B.Cu) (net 3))
 (segment (start 125.095 119.38) (end 125.095 114.935) (width 0.25) (layer B.Cu) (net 3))
 (segment (start 125.095 114.935) (end 127 113.03) (width 0.25) (layer B.Cu) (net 3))
 (segment (start 127 107.95) (end 125.095 106.045) (width 0.25) (layer B.Cu) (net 3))
 (segment (start 127 113.03) (end 127 107.95) (width 0.25) (layer B.Cu) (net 3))
 (segment (start 140.335 101.115) (end 140.335 116.84) (width 0.25) (layer B.Cu) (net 3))
 (segment (start 133.275 123.9) (end 129.94 123.9) (width 0.25) (layer B.Cu) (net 3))
 (segment (start 140.335 116.84) (end 133.275 123.9) (width 0.25) (layer B.Cu) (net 3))
 (segment (start 140.335 101.115) (end 143.36 104.14) (width 0.25) (layer F.Cu) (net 3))
 (segment (start 149.7116 104.14) (end 149.9362 103.9154) (width 0.25) (layer F.Cu) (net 3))
 (segment (start 143.36 104.14) (end 149.7116 104.14) (width 0.25) (layer F.Cu) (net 3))
 (segment (start 140.335 98.425) (end 144.145 94.615) (width 0.25) (layer F.Cu) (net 3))
 (segment (start 140.335 101.115) (end 140.335 98.425) (width 0.25) (layer F.Cu) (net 3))
 (segment (start 137.795 101.115) (end 137.795 103.505) (width 0.25) (layer F.Cu) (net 2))
 (segment (start 140.7454 106.4554) (end 149.9362 106.4554) (width 0.25) (layer F.Cu) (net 2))
 (segment (start 137.795 103.505) (end 140.7454 106.4554) (width 0.25) (layer F.Cu) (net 2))
 (segment (start 137.795 101.115) (end 137.31 101.115) (width 0.25) (layer F.Cu) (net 2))
 (segment (start 137.31 101.115) (end 131.445 95.25) (width 0.25) (layer F.Cu) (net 2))
 (segment (start 114.935 84.455) (end 114.935 86.995) (width 0.25) (layer B.Cu) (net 4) (status 30))
 (segment (start 129.94 113.74) (end 128.195 113.74) (width 0.25) (layer F.Cu) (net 4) (status 10))
 (segment (start 128.195 113.74) (end 127.635 114.3) (width 0.25) (layer F.Cu) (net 4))
 (segment (start 127.635 114.3) (end 127.635 121.92) (width 0.25) (layer F.Cu) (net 4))
 (segment (start 127.635 121.92) (end 127 122.555) (width 0.25) (layer F.Cu) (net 4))
 (segment (start 105.885 122.555) (end 104.54 123.9) (width 0.25) (layer F.Cu) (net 4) (status 20))
 (segment (start 127 122.555) (end 105.885 122.555) (width 0.25) (layer F.Cu) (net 4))
 (segment (start 142.875 101.115) (end 142.875 111.76) (width 0.25) (layer B.Cu) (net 4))
 (segment (start 142.875 111.76) (end 142.875 111.76) (width 0.25) (layer B.Cu) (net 4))
 (via (at 142.875 111.76) (size 0.8) (drill 0.4) (layers F.Cu B.Cu) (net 4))
 (segment (start 142.875 111.76) (end 142.875 112.395) (width 0.25) (layer F.Cu) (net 4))
 (segment (start 141.53 113.74) (end 129.94 113.74) (width 0.25) (layer F.Cu) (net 4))
 (segment (start 142.875 112.395) (end 141.53 113.74) (width 0.25) (layer F.Cu) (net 4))
 (segment (start 148.855 101.115) (end 163.83 86.14) (width 0.25) (layer B.Cu) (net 4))
 (segment (start 163.83 86.14) (end 163.83 85.09) (width 0.25) (layer B.Cu) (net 4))
 (segment (start 142.875 101.115) (end 148.855 101.115) (width 0.25) (layer B.Cu) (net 4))
 (segment (start 142.875 99.06) (end 142.875 101.115) (width 0.25) (layer B.Cu) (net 4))
 (segment (start 126.365 82.55) (end 142.875 99.06) (width 0.25) (layer B.Cu) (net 4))
 (segment (start 119.38 82.55) (end 126.365 82.55) (width 0.25) (layer B.Cu) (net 4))
 (segment (start 117.475 84.455) (end 119.38 82.55) (width 0.25) (layer B.Cu) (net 4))
 (segment (start 114.935 84.455) (end 117.475 84.455) (width 0.25) (layer B.Cu) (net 4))
 (segment (start 109.855 119.38) (end 110.49 119.38) (width 0.25) (layer B.Cu) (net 5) (status 30))
 (segment (start 109.855 119.38) (end 107.95 117.475) (width 0.25) (layer B.Cu) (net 5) (status 10))
 (segment (start 107.95 117.475) (end 107.315 116.84) (width 0.25) (layer B.Cu) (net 5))
 (segment (start 107.315 116.84) (end 107.315 104.775) (width 0.25) (layer B.Cu) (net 5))
 (segment (start 107.315 104.775) (end 108.585 103.505) (width 0.25) (layer B.Cu) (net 5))
 (segment (start 108.585 103.505) (end 109.22 102.87) (width 0.25) (layer B.Cu) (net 5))
 (segment (start 109.22 102.87) (end 113.665 102.87) (width 0.25) (layer B.Cu) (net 5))
 (via (at 113.665 102.87) (size 0.8) (drill 0.4) (layers F.Cu B.Cu) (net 5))
 (segment (start 129.23 102.87) (end 129.94 103.58) (width 0.25) (layer F.Cu) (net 5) (status 30))
 (segment (start 113.665 102.87) (end 129.23 102.87) (width 0.25) (layer F.Cu) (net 5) (status 20))
 (segment (start 118.745 97.155) (end 118.745 118.11) (width 0.25) (layer B.Cu) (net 9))
 (segment (start 122.555 93.345) (end 118.745 97.155) (width 0.25) (layer B.Cu) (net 9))
 (segment (start 118.745 118.11) (end 120.015 119.38) (width 0.25) (layer B.Cu) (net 9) (status 20))
 (segment (start 122.555 86.995) (end 122.555 93.345) (width 0.25) (layer B.Cu) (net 9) (status 10))
 (segment (start 122.555 84.455) (end 121.285 84.455) (width 0.25) (layer B.Cu) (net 10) (status 10))
 (segment (start 121.285 84.455) (end 116.205 89.535) (width 0.25) (layer B.Cu) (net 10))
 (segment (start 116.205 115.57) (end 112.395 119.38) (width 0.25) (layer B.Cu) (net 10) (status 20))
 (segment (start 116.205 89.535) (end 116.205 115.57) (width 0.25) (layer B.Cu) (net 10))
 (segment (start 120.65 135.255) (end 120.65 125.095) (width 0.25) (layer F.Cu) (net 13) (status 10))
 (via (at 120.65 125.095) (size 0.8) (drill 0.4) (layers F.Cu B.Cu) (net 13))
 (segment (start 120.65 125.095) (end 116.205 120.65) (width 0.25) (layer B.Cu) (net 13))
 (segment (start 116.205 120.65) (end 116.205 117.475) (width 0.25) (layer B.Cu) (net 13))
 (via (at 116.205 117.475) (size 0.8) (drill 0.4) (layers F.Cu B.Cu) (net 13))
 (segment (start 116.205 117.475) (end 116.205 115.57) (width 0.25) (layer F.Cu) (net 13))
 (segment (start 116.205 115.57) (end 113.665 113.03) (width 0.25) (layer F.Cu) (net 13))
 (segment (start 113.665 113.03) (end 113.665 110.49) (width 0.25) (layer F.Cu) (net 13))
 (segment (start 113.665 110.49) (end 113.665 109.855) (width 0.25) (layer F.Cu) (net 13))
 (via (at 113.665 109.855) (size 0.8) (drill 0.4) (layers F.Cu B.Cu) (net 13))
 (segment (start 113.665 107.315) (end 114.935 106.045) (width 0.25) (layer B.Cu) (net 13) (status 20))
 (segment (start 113.665 109.855) (end 113.665 107.315) (width 0.25) (layer B.Cu) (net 13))
 (segment (start 117.475 119.38) (end 127 128.905) (width 0.25) (layer B.Cu) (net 1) (status 10))
 (segment (start 137.6466 128.905) (end 136.525 128.905) (width 0.25) (layer B.Cu) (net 1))
 (segment (start 149.9362 116.6154) (end 137.6466 128.905) (width 0.25) (layer B.Cu) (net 1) (status 10))
 (segment (start 127 128.905) (end 136.525 128.905) (width 0.25) (layer B.Cu) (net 1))
 (segment (start 111.125 115.57) (end 114.935 119.38) (width 0.25) (layer F.Cu) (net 11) (status 20))
 (segment (start 111.125 109.855) (end 111.125 115.57) (width 0.25) (layer F.Cu) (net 11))
 (segment (start 109.855 108.585) (end 111.125 109.855) (width 0.25) (layer F.Cu) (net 11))
 (segment (start 109.855 106.045) (end 109.855 108.585) (width 0.25) (layer F.Cu) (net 11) (status 10))
 (segment (start 122.555 117.475) (end 122.555 119.38) (width 0.25) (layer F.Cu) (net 12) (status 20))
 (segment (start 121.285 116.205) (end 122.555 117.475) (width 0.25) (layer F.Cu) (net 12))
 (segment (start 121.285 110.49) (end 121.285 116.205) (width 0.25) (layer F.Cu) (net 12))
 (segment (start 120.65 109.855) (end 121.285 110.49) (width 0.25) (layer F.Cu) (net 12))
 (segment (start 116.205 109.855) (end 120.65 109.855) (width 0.25) (layer F.Cu) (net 12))
 (segment (start 112.395 106.045) (end 116.205 109.855) (width 0.25) (layer F.Cu) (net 12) (status 10))
 (segment (start 108.585 126.365) (end 107.95 126.365) (width 0.25) (layer F.Cu) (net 14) (status 30))
 (segment (start 107.95 126.365) (end 106.68 127.635) (width 0.25) (layer F.Cu) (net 14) (status 10))
 (segment (start 106.68 127.635) (end 106.68 130.81) (width 0.25) (layer F.Cu) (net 14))
 (segment (start 111.125 135.255) (end 113.03 135.255) (width 0.25) (layer F.Cu) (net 14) (status 20))
 (segment (start 106.68 130.81) (end 111.125 135.255) (width 0.25) (layer F.Cu) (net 14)))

